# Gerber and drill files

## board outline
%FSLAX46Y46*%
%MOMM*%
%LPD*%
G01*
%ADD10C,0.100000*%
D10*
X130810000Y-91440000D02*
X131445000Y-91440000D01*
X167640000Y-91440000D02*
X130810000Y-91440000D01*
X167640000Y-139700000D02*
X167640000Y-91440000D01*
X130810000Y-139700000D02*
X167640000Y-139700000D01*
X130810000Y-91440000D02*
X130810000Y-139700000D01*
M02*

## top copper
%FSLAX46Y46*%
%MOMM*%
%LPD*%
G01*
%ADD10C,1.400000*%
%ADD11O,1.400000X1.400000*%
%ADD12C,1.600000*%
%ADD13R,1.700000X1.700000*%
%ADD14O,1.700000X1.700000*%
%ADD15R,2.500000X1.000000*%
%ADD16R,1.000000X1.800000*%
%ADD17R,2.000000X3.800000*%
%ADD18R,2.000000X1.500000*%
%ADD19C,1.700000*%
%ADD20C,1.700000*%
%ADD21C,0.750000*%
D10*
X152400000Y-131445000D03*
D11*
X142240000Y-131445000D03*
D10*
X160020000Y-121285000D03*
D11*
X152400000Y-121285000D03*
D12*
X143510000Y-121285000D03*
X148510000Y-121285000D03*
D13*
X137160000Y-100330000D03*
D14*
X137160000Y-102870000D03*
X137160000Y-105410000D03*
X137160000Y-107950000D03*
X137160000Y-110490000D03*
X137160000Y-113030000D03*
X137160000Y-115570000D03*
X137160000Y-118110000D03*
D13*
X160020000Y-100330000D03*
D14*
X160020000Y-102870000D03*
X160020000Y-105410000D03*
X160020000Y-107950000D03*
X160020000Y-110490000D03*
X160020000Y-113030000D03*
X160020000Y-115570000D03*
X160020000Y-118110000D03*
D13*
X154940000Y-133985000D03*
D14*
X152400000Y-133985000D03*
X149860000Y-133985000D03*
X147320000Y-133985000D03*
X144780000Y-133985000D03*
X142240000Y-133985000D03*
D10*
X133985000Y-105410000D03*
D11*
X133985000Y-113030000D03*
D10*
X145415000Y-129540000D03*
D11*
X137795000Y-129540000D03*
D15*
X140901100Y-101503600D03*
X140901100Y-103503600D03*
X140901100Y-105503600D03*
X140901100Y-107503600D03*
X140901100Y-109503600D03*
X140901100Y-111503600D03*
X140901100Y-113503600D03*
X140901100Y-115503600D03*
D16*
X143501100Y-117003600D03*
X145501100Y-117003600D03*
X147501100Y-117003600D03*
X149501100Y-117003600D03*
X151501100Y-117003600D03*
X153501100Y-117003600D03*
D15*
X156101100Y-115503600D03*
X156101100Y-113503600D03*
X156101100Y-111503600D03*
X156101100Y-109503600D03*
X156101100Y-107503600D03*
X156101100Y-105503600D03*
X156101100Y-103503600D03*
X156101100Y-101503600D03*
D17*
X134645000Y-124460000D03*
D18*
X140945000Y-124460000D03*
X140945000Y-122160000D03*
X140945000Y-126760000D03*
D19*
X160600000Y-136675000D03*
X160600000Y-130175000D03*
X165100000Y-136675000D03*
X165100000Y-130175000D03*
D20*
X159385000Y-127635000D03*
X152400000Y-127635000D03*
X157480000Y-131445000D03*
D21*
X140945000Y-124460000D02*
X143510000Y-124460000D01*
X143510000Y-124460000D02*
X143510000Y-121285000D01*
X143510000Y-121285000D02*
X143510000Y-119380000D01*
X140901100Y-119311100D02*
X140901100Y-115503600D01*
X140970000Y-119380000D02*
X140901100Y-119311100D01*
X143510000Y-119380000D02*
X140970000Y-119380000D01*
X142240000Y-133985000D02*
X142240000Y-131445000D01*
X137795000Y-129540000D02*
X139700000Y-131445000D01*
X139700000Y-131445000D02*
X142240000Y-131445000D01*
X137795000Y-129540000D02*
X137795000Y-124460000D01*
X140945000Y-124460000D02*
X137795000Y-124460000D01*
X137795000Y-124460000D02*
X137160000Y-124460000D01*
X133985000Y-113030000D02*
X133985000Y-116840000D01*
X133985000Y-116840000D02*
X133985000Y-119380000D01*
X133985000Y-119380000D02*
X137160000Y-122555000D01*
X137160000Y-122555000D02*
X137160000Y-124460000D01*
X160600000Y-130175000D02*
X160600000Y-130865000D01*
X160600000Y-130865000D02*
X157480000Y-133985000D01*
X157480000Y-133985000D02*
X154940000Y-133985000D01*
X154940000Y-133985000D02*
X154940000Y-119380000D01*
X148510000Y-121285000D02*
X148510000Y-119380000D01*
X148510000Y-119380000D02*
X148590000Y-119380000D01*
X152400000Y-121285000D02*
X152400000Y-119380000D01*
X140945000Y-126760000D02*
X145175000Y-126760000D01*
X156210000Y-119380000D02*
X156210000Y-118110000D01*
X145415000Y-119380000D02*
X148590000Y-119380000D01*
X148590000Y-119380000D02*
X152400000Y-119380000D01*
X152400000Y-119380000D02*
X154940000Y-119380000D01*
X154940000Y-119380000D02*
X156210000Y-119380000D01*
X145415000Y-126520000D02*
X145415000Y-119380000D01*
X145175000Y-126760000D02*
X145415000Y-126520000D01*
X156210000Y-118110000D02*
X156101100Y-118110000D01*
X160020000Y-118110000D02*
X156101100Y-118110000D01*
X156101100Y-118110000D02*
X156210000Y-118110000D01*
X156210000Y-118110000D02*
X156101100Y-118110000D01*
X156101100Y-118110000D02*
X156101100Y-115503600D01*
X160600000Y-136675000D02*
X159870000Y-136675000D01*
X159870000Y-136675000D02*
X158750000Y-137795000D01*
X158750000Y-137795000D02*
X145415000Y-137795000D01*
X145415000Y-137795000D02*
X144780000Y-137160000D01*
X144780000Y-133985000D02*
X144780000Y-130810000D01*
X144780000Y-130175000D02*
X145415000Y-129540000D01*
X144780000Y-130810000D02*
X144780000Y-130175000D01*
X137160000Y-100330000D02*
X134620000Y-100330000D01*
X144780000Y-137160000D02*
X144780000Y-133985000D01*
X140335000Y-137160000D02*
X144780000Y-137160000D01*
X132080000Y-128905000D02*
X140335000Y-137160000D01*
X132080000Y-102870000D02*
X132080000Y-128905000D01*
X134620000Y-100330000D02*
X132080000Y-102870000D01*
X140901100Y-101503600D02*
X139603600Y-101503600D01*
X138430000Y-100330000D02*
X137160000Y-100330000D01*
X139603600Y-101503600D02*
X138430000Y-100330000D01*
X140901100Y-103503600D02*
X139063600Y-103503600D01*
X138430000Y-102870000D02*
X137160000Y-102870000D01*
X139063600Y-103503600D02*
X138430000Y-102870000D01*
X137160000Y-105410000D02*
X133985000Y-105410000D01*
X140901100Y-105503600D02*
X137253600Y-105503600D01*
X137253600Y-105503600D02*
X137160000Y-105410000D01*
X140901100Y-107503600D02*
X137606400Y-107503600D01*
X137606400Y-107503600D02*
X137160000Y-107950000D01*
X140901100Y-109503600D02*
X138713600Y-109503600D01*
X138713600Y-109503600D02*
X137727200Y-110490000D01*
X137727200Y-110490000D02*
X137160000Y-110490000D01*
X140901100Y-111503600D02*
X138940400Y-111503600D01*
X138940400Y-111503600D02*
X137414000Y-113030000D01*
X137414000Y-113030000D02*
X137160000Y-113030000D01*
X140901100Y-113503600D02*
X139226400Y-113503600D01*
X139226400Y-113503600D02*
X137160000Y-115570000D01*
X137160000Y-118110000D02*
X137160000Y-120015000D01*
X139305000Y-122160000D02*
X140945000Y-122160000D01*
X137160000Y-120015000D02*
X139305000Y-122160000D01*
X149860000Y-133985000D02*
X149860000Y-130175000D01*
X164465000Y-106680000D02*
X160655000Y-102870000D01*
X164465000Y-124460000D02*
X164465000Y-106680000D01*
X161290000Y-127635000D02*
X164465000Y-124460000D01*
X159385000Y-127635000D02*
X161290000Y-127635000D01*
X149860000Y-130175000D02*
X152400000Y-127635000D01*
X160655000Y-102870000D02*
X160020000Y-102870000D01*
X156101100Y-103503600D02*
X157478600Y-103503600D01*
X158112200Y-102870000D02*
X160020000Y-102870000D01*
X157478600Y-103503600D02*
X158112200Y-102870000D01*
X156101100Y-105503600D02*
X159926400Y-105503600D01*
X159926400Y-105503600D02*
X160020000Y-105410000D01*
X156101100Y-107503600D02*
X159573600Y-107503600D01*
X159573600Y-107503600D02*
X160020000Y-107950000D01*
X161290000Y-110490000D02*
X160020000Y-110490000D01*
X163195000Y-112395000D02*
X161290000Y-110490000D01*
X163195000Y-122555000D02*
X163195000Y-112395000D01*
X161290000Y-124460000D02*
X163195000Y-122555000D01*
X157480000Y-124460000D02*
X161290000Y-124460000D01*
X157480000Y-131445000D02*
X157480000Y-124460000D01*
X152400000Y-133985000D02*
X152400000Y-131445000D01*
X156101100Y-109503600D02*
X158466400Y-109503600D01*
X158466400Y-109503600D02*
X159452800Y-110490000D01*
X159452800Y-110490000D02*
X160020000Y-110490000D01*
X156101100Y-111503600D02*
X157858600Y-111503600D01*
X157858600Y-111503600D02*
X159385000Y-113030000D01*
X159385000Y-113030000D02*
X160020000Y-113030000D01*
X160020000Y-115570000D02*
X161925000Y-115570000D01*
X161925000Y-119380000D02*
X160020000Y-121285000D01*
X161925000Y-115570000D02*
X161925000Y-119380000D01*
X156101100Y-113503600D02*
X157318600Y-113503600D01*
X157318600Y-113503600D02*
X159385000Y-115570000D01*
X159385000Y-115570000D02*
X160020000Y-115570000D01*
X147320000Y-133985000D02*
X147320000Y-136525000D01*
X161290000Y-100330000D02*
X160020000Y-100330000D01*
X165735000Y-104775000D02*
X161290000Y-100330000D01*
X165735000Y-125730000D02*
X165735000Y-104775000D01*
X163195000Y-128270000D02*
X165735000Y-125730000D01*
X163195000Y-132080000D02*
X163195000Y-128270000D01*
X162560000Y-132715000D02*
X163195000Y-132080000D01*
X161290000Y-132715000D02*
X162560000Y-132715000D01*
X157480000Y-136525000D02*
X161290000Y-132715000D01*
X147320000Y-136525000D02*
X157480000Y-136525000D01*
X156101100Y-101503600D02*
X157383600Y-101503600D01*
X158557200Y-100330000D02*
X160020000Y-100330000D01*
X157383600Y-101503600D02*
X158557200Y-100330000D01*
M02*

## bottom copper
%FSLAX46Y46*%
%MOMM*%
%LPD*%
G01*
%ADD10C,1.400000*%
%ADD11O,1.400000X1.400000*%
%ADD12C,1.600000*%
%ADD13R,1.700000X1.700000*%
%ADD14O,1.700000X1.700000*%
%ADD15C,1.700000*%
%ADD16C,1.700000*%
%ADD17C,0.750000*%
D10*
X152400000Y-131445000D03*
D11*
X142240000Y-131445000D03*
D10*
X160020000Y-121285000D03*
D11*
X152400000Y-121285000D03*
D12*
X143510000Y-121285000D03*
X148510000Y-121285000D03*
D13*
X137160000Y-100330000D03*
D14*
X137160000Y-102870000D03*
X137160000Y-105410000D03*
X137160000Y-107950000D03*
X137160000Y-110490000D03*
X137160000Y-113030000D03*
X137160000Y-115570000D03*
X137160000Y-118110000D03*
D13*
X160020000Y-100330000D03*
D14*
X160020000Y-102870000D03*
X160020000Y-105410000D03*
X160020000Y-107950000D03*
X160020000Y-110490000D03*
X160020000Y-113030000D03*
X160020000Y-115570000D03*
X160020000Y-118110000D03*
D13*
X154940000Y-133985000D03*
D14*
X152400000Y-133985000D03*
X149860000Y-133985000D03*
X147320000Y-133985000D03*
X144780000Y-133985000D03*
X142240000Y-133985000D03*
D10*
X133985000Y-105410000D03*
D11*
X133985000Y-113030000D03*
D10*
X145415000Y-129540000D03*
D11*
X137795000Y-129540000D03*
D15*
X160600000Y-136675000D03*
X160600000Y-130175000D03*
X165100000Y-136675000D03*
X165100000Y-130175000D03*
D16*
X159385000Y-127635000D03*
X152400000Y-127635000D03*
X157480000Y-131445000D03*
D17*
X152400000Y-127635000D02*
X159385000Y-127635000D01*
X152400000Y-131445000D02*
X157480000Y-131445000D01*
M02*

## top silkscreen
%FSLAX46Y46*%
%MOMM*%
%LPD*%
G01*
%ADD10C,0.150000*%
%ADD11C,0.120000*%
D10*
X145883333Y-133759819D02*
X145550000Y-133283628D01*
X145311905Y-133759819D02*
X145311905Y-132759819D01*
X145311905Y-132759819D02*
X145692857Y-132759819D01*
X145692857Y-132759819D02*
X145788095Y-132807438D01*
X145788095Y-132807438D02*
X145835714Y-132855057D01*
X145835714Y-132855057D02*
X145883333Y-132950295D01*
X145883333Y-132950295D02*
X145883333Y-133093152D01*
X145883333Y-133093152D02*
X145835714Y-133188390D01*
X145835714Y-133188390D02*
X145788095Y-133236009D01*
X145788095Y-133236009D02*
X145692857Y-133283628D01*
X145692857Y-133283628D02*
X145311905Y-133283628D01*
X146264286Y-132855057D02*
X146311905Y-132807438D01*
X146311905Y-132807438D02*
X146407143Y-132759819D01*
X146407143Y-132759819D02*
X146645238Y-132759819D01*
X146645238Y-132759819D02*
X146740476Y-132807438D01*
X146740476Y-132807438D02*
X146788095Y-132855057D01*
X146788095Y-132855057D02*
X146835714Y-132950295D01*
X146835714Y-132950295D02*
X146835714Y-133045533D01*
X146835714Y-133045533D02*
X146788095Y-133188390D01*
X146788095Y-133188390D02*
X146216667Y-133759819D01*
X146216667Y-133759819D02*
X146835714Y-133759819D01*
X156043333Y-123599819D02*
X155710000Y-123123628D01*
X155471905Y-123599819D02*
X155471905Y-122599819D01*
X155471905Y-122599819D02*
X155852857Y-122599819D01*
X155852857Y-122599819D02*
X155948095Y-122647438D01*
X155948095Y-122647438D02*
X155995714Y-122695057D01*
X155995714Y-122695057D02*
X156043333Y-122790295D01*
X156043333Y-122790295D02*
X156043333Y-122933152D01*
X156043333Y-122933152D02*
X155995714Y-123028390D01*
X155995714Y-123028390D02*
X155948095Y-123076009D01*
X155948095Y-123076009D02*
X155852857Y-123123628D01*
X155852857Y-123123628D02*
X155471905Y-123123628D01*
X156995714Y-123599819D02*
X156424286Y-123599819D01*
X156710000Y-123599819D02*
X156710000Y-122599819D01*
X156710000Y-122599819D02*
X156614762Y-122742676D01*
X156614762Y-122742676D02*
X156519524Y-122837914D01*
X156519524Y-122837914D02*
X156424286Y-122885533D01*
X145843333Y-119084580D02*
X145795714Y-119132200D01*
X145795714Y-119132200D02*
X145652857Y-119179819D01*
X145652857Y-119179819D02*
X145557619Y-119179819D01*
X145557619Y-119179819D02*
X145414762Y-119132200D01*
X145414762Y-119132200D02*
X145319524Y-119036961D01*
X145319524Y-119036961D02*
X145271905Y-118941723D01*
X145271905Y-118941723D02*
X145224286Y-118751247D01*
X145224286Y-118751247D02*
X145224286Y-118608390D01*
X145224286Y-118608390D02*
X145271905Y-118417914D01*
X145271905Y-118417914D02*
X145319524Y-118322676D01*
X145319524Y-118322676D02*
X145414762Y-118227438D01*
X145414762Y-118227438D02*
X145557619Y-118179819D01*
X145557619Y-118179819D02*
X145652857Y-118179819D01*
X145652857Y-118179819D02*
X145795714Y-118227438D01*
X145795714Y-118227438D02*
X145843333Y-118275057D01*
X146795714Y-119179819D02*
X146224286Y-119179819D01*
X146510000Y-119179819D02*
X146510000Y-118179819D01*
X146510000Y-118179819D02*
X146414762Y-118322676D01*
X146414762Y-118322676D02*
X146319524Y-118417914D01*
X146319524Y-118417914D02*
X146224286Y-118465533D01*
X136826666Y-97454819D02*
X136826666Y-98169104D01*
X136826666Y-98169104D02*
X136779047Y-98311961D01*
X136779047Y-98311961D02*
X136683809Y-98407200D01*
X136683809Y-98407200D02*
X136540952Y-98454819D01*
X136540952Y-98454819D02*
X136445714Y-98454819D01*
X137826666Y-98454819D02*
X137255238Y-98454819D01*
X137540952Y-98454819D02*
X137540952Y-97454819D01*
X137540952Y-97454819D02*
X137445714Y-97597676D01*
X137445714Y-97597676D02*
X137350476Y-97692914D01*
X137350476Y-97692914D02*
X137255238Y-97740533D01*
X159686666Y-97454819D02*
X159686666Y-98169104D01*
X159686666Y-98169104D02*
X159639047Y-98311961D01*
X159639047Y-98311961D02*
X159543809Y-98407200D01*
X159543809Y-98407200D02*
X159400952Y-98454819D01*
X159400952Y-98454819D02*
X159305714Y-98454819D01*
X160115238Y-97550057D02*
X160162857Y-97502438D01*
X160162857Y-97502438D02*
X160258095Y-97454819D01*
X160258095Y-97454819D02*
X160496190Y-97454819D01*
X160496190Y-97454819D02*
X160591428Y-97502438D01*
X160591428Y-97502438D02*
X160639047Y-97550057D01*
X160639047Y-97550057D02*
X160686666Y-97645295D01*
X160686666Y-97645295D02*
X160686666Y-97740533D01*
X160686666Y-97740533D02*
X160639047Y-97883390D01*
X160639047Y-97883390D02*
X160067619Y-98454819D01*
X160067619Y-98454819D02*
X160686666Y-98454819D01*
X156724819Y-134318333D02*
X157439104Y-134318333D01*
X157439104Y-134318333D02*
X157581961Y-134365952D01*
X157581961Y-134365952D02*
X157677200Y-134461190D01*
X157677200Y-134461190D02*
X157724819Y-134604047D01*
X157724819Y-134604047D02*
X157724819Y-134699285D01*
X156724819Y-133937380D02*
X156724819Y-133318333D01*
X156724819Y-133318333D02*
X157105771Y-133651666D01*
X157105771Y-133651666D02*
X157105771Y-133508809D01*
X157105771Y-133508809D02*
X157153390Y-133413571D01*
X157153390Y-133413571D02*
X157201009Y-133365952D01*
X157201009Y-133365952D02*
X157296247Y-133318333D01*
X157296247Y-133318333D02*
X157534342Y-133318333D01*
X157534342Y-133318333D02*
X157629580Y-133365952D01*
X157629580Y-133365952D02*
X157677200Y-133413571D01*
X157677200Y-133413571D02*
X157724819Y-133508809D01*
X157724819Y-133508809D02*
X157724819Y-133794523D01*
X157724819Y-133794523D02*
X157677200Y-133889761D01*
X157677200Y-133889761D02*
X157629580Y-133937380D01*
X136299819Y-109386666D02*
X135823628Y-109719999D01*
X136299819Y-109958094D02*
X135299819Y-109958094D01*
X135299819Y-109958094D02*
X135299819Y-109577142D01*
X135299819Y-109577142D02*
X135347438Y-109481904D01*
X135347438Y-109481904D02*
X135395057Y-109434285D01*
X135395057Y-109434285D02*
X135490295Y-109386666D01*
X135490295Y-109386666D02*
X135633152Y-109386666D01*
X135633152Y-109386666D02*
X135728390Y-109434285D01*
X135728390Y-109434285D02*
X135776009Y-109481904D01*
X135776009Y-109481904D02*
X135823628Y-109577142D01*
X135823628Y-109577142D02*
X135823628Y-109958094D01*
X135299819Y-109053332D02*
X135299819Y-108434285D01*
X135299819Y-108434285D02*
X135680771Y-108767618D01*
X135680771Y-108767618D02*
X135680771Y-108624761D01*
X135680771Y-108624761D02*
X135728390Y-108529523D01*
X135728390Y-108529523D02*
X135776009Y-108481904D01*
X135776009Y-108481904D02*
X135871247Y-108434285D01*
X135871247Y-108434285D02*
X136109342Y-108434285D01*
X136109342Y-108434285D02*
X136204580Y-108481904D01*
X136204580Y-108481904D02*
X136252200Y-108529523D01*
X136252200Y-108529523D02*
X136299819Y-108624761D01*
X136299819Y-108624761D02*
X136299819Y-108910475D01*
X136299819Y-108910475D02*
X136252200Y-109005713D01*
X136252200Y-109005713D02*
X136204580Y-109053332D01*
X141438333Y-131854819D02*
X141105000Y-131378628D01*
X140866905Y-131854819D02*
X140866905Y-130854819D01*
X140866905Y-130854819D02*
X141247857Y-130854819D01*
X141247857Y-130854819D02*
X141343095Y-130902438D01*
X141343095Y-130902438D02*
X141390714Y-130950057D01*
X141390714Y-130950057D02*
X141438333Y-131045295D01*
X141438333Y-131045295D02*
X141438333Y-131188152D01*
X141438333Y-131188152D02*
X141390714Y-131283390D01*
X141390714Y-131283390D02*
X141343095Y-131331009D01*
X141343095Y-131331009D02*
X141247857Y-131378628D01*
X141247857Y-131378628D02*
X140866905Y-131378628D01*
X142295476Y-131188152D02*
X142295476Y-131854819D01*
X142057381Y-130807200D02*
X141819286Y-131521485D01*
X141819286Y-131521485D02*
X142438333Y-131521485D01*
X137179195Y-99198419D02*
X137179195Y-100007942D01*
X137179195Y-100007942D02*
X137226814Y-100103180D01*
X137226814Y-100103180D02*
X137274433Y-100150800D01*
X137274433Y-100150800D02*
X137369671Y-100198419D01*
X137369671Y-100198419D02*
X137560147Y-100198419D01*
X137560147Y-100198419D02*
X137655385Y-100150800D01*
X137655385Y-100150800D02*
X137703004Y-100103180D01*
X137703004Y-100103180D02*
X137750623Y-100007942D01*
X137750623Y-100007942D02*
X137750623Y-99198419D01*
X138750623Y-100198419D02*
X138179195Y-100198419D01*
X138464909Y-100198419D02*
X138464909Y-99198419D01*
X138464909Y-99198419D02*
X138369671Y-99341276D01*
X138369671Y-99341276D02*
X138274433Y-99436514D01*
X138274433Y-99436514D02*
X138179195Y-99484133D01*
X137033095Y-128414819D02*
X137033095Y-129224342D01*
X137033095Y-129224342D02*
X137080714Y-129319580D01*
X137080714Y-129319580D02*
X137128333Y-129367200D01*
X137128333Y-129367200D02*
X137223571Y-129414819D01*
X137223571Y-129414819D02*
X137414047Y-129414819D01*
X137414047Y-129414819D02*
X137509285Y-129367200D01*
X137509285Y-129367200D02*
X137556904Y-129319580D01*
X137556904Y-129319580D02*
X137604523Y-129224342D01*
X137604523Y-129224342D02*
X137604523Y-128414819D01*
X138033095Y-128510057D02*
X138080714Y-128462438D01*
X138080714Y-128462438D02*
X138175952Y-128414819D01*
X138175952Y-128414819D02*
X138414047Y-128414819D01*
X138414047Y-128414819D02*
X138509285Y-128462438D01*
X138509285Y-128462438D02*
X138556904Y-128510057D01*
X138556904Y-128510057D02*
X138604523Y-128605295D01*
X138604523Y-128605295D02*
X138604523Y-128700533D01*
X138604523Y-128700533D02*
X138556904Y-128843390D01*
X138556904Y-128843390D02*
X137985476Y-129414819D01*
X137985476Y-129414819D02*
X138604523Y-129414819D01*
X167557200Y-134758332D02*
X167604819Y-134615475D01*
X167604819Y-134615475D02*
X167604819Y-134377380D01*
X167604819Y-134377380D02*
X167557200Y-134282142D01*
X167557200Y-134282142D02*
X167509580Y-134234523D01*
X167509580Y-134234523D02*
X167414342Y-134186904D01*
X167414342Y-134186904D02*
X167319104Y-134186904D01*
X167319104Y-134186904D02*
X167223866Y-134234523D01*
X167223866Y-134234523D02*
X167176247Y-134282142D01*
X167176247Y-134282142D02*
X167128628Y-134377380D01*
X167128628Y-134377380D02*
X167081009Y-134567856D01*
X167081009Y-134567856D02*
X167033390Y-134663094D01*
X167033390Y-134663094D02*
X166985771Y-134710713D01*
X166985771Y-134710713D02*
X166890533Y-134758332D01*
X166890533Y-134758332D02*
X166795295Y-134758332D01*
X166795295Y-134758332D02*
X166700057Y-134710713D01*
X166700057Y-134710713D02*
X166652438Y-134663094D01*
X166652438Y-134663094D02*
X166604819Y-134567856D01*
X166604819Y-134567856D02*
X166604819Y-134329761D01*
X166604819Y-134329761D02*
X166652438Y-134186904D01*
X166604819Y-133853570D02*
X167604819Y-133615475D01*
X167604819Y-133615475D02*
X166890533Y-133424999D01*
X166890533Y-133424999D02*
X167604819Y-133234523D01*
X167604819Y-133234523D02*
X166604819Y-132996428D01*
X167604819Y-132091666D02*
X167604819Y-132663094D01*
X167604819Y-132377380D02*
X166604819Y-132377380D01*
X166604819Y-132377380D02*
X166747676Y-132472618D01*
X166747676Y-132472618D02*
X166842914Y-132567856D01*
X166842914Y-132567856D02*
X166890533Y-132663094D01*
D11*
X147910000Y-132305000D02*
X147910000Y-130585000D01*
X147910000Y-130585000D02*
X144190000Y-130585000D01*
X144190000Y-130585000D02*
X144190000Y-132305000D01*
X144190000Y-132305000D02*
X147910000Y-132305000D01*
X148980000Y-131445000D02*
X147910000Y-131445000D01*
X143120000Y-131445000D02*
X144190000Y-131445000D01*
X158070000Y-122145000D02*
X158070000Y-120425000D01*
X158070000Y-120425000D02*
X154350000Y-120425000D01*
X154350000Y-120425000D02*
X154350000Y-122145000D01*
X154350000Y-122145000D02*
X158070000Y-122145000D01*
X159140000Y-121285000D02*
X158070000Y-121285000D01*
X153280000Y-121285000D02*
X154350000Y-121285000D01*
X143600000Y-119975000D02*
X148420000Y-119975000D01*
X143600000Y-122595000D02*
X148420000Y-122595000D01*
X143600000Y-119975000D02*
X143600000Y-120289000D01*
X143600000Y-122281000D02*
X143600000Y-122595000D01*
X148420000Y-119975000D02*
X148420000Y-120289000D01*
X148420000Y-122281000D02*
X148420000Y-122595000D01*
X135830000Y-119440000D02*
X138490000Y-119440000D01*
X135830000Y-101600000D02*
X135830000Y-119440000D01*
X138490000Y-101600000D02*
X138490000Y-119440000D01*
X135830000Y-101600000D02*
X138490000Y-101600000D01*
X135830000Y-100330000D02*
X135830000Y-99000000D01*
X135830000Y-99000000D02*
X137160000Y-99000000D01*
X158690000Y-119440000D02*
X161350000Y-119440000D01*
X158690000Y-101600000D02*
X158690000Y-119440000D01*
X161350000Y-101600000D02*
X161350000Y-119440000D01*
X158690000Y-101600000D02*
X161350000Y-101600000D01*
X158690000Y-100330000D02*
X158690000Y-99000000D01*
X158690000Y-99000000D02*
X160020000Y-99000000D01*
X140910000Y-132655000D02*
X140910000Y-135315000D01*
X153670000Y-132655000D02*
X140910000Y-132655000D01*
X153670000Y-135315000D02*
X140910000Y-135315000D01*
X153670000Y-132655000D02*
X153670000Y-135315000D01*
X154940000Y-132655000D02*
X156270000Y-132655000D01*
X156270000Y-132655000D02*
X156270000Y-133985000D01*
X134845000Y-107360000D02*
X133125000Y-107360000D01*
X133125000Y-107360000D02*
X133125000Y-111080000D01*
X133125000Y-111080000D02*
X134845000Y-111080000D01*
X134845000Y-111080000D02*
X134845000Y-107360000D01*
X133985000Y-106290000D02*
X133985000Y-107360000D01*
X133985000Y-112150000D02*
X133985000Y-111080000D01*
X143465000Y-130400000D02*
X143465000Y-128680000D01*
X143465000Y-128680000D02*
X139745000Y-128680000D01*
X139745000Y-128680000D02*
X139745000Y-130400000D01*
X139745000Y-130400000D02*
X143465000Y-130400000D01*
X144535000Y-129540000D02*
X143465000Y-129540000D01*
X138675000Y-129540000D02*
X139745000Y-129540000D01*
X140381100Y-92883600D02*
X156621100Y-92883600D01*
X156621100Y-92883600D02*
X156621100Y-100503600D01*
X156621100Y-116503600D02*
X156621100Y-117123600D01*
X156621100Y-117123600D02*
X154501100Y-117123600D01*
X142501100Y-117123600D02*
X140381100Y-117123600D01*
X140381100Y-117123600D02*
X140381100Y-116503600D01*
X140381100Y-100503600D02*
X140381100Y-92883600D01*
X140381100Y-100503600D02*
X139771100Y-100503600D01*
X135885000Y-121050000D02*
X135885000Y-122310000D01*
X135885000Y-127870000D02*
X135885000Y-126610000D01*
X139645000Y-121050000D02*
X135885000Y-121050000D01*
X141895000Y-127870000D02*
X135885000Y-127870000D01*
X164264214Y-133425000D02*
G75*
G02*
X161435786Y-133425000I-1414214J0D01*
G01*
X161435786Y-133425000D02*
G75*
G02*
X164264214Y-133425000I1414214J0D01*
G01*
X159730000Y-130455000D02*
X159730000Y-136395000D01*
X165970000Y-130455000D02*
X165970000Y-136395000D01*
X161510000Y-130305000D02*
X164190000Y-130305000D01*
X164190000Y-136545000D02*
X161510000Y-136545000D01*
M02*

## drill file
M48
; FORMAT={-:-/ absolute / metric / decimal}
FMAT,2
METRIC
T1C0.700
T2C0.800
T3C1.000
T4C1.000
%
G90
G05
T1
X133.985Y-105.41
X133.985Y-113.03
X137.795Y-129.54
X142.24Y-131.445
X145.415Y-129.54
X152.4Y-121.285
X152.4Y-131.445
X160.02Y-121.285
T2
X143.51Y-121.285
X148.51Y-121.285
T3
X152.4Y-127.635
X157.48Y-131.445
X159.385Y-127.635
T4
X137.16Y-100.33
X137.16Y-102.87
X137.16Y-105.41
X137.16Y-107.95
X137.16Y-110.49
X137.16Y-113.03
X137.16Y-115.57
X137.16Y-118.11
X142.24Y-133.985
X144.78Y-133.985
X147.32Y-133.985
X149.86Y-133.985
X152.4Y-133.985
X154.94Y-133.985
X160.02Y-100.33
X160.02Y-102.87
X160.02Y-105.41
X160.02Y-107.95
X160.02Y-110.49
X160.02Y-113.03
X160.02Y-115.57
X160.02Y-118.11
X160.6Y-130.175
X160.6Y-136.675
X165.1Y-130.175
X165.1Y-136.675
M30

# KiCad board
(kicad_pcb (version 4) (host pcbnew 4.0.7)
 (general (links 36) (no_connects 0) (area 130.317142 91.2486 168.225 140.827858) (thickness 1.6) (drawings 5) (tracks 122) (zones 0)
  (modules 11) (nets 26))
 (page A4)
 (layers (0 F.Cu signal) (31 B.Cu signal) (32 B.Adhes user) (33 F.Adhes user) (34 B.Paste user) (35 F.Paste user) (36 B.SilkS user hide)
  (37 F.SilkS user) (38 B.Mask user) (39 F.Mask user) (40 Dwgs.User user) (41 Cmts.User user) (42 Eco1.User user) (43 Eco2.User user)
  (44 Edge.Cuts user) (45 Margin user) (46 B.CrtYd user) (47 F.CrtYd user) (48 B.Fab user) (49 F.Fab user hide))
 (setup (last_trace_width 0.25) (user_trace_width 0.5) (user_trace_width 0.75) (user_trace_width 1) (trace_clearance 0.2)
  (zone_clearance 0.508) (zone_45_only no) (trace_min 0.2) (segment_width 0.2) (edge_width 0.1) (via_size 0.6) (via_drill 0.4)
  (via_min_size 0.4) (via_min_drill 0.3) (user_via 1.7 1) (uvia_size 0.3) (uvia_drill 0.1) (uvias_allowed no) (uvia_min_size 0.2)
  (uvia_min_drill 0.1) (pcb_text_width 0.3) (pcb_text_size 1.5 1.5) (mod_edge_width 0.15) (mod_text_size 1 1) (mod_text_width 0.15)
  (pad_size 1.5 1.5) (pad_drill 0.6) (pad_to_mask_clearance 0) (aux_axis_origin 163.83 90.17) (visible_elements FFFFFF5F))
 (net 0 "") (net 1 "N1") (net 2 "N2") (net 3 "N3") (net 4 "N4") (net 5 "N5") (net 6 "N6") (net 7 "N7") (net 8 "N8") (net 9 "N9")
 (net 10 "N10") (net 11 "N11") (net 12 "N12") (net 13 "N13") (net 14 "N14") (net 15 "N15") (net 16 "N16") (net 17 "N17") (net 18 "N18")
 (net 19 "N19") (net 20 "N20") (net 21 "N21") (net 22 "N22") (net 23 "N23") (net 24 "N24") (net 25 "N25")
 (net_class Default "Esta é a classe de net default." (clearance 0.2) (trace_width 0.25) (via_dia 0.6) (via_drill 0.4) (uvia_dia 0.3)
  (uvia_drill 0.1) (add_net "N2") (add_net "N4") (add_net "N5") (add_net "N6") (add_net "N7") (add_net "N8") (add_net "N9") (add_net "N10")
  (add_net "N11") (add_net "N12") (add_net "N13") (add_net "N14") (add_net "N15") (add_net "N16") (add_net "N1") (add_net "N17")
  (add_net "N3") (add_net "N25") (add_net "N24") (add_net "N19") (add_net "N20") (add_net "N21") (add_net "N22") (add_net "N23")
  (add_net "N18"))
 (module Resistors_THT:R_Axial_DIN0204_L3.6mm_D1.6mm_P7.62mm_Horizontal (layer F.Cu) (at 149.86 131.445 180)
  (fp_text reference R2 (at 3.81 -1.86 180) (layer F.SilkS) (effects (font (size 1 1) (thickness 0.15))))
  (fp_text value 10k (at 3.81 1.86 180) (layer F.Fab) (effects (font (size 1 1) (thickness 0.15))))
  (fp_line (start 1.95 -0.86) (end 1.95 0.86) (layer F.SilkS) (width 0.12))
  (fp_line (start 1.95 0.86) (end 5.67 0.86) (layer F.SilkS) (width 0.12))
  (fp_line (start 5.67 0.86) (end 5.67 -0.86) (layer F.SilkS) (width 0.12))
  (fp_line (start 5.67 -0.86) (end 1.95 -0.86) (layer F.SilkS) (width 0.12))
  (fp_line (start 0.88 0) (end 1.95 0) (layer F.SilkS) (width 0.12))
  (fp_line (start 6.74 0) (end 5.67 0) (layer F.SilkS) (width 0.12))
  (pad 1 thru_hole circle (at -2.54 0 180) (size 1.4 1.4) (drill 0.7) (layers *.Cu *.Mask) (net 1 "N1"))
  (pad 2 thru_hole oval (at 7.62 0 180) (size 1.4 1.4) (drill 0.7) (layers *.Cu *.Mask) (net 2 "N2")))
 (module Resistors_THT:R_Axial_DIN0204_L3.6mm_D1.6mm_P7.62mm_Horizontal (layer F.Cu) (at 160.02 121.285 180)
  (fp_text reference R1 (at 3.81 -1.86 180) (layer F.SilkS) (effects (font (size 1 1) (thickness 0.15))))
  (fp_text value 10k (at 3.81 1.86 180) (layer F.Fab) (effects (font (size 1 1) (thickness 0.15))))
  (fp_line (start 1.95 -0.86) (end 1.95 0.86) (layer F.SilkS) (width 0.12))
  (fp_line (start 1.95 0.86) (end 5.67 0.86) (layer F.SilkS) (width 0.12))
  (fp_line (start 5.67 0.86) (end 5.67 -0.86) (layer F.SilkS) (width 0.12))
  (fp_line (start 5.67 -0.86) (end 1.95 -0.86) (layer F.SilkS) (width 0.12))
  (fp_line (start 0.88 0) (end 1.95 0) (layer F.SilkS) (width 0.12))
  (fp_line (start 6.74 0) (end 5.67 0) (layer F.SilkS) (width 0.12))
  (pad 1 thru_hole circle (at 0 0 180) (size 1.4 1.4) (drill 0.7) (layers *.Cu *.Mask) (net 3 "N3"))
  (pad 2 thru_hole oval (at 7.62 0 180) (size 1.4 1.4) (drill 0.7) (layers *.Cu *.Mask) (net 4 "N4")))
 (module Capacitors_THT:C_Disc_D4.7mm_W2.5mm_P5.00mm (layer F.Cu) (at 143.51 121.285)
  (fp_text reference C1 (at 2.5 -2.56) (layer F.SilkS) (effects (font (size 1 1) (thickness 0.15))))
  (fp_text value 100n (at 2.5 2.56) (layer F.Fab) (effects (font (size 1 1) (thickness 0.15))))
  (fp_line (start 0.09 -1.31) (end 4.91 -1.31) (layer F.SilkS) (width 0.12))
  (fp_line (start 0.09 1.31) (end 4.91 1.31) (layer F.SilkS) (width 0.12))
  (fp_line (start 0.09 -1.31) (end 0.09 -0.996) (layer F.SilkS) (width 0.12))
  (fp_line (start 0.09 0.996) (end 0.09 1.31) (layer F.SilkS) (width 0.12))
  (fp_line (start 4.91 -1.31) (end 4.91 -0.996) (layer F.SilkS) (width 0.12))
  (fp_line (start 4.91 0.996) (end 4.91 1.31) (layer F.SilkS) (width 0.12))
  (pad 1 thru_hole circle (at 0 0) (size 1.6 1.6) (drill 0.8) (layers *.Cu *.Mask) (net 2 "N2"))
  (pad 2 thru_hole circle (at 5 0) (size 1.6 1.6) (drill 0.8) (layers *.Cu *.Mask) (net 4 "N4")))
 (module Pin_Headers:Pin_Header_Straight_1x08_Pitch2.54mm (layer F.Cu) (at 137.16 100.33)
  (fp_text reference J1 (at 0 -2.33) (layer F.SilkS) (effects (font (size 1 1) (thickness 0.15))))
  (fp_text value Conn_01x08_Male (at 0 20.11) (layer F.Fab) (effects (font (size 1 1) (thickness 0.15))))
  (fp_line (start -1.33 19.11) (end 1.33 19.11) (layer F.SilkS) (width 0.12))
  (fp_line (start -1.33 1.27) (end -1.33 19.11) (layer F.SilkS) (width 0.12))
  (fp_line (start 1.33 1.27) (end 1.33 19.11) (layer F.SilkS) (width 0.12))
  (fp_line (start -1.33 1.27) (end 1.33 1.27) (layer F.SilkS) (width 0.12))
  (fp_line (start -1.33 0) (end -1.33 -1.33) (layer F.SilkS) (width 0.12))
  (fp_line (start -1.33 -1.33) (end 0 -1.33) (layer F.SilkS) (width 0.12))
  (pad 1 thru_hole rect (at 0 0) (size 1.7 1.7) (drill 1) (layers *.Cu *.Mask) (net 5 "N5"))
  (pad 2 thru_hole oval (at 0 2.54) (size 1.7 1.7) (drill 1) (layers *.Cu *.Mask) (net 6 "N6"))
  (pad 3 thru_hole oval (at 0 5.08) (size 1.7 1.7) (drill 1) (layers *.Cu *.Mask) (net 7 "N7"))
  (pad 4 thru_hole oval (at 0 7.62) (size 1.7 1.7) (drill 1) (layers *.Cu *.Mask) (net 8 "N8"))
  (pad 5 thru_hole oval (at 0 10.16) (size 1.7 1.7) (drill 1) (layers *.Cu *.Mask) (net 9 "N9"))
  (pad 6 thru_hole oval (at 0 12.7) (size 1.7 1.7) (drill 1) (layers *.Cu *.Mask) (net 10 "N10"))
  (pad 7 thru_hole oval (at 0 15.24) (size 1.7 1.7) (drill 1) (layers *.Cu *.Mask) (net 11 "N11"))
  (pad 8 thru_hole oval (at 0 17.78) (size 1.7 1.7) (drill 1) (layers *.Cu *.Mask) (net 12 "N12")))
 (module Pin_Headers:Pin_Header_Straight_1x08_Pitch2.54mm (layer F.Cu) (at 160.02 100.33)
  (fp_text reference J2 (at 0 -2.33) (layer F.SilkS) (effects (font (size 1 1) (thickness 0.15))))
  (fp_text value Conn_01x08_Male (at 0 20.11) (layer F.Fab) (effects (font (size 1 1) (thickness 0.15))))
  (fp_line (start -1.33 19.11) (end 1.33 19.11) (layer F.SilkS) (width 0.12))
  (fp_line (start -1.33 1.27) (end -1.33 19.11) (layer F.SilkS) (width 0.12))
  (fp_line (start 1.33 1.27) (end 1.33 19.11) (layer F.SilkS) (width 0.12))
  (fp_line (start -1.33 1.27) (end 1.33 1.27) (layer F.SilkS) (width 0.12))
  (fp_line (start -1.33 0) (end -1.33 -1.33) (layer F.SilkS) (width 0.12))
  (fp_line (start -1.33 -1.33) (end 0 -1.33) (layer F.SilkS) (width 0.12))
  (pad 1 thru_hole rect (at 0 0) (size 1.7 1.7) (drill 1) (layers *.Cu *.Mask) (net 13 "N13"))
  (pad 2 thru_hole oval (at 0 2.54) (size 1.7 1.7) (drill 1) (layers *.Cu *.Mask) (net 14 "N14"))
  (pad 3 thru_hole oval (at 0 5.08) (size 1.7 1.7) (drill 1) (layers *.Cu *.Mask) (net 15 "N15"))
  (pad 4 thru_hole oval (at 0 7.62) (size 1.7 1.7) (drill 1) (layers *.Cu *.Mask) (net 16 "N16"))
  (pad 5 thru_hole oval (at 0 10.16) (size 1.7 1.7) (drill 1) (layers *.Cu *.Mask) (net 1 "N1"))
  (pad 6 thru_hole oval (at 0 12.7) (size 1.7 1.7) (drill 1) (layers *.Cu *.Mask) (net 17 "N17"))
  (pad 7 thru_hole oval (at 0 15.24) (size 1.7 1.7) (drill 1) (layers *.Cu *.Mask) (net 3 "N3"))
  (pad 8 thru_hole oval (at 0 17.78) (size 1.7 1.7) (drill 1) (layers *.Cu *.Mask) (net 4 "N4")))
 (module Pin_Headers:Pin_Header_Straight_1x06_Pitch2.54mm (layer F.Cu) (at 154.94 133.985 270)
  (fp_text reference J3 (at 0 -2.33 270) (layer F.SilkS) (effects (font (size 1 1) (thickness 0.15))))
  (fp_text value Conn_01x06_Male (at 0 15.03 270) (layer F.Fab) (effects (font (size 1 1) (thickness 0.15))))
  (fp_line (start -1.33 14.03) (end 1.33 14.03) (layer F.SilkS) (width 0.12))
  (fp_line (start -1.33 1.27) (end -1.33 14.03) (layer F.SilkS) (width 0.12))
  (fp_line (start 1.33 1.27) (end 1.33 14.03) (layer F.SilkS) (width 0.12))
  (fp_line (start -1.33 1.27) (end 1.33 1.27) (layer F.SilkS) (width 0.12))
  (fp_line (start -1.33 0) (end -1.33 -1.33) (layer F.SilkS) (width 0.12))
  (fp_line (start -1.33 -1.33) (end 0 -1.33) (layer F.SilkS) (width 0.12))
  (pad 1 thru_hole rect (at 0 0 270) (size 1.7 1.7) (drill 1) (layers *.Cu *.Mask) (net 4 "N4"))
  (pad 2 thru_hole oval (at 0 2.54 270) (size 1.7 1.7) (drill 1) (layers *.Cu *.Mask) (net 1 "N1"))
  (pad 3 thru_hole oval (at 0 5.08 270) (size 1.7 1.7) (drill 1) (layers *.Cu *.Mask) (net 14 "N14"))
  (pad 4 thru_hole oval (at 0 7.62 270) (size 1.7 1.7) (drill 1) (layers *.Cu *.Mask) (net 13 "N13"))
  (pad 5 thru_hole oval (at 0 10.16 270) (size 1.7 1.7) (drill 1) (layers *.Cu *.Mask) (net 5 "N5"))
  (pad 6 thru_hole oval (at 0 12.7 270) (size 1.7 1.7) (drill 1) (layers *.Cu *.Mask) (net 2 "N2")))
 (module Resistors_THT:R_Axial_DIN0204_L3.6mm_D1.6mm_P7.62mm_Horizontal (layer F.Cu) (at 133.985 105.41 270)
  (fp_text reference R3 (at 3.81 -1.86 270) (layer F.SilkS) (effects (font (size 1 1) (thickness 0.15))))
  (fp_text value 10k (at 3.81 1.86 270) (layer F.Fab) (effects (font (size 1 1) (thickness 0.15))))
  (fp_line (start 1.95 -0.86) (end 1.95 0.86) (layer F.SilkS) (width 0.12))
  (fp_line (start 1.95 0.86) (end 5.67 0.86) (layer F.SilkS) (width 0.12))
  (fp_line (start 5.67 0.86) (end 5.67 -0.86) (layer F.SilkS) (width 0.12))
  (fp_line (start 5.67 -0.86) (end 1.95 -0.86) (layer F.SilkS) (width 0.12))
  (fp_line (start 0.88 0) (end 1.95 0) (layer F.SilkS) (width 0.12))
  (fp_line (start 6.74 0) (end 5.67 0) (layer F.SilkS) (width 0.12))
  (pad 1 thru_hole circle (at 0 0 270) (size 1.4 1.4) (drill 0.7) (layers *.Cu *.Mask) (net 7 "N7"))
  (pad 2 thru_hole oval (at 7.62 0 270) (size 1.4 1.4) (drill 0.7) (layers *.Cu *.Mask) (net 2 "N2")))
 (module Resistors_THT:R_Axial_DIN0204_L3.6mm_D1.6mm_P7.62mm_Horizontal (layer F.Cu) (at 145.415 129.54 180)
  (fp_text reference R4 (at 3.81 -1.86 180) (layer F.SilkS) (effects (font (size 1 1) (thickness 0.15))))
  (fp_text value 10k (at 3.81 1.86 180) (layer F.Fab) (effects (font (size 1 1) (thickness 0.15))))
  (fp_line (start 1.95 -0.86) (end 1.95 0.86) (layer F.SilkS) (width 0.12))
  (fp_line (start 1.95 0.86) (end 5.67 0.86) (layer F.SilkS) (width 0.12))
  (fp_line (start 5.67 0.86) (end 5.67 -0.86) (layer F.SilkS) (width 0.12))
  (fp_line (start 5.67 -0.86) (end 1.95 -0.86) (layer F.SilkS) (width 0.12))
  (fp_line (start 0.88 0) (end 1.95 0) (layer F.SilkS) (width 0.12))
  (fp_line (start 6.74 0) (end 5.67 0) (layer F.SilkS) (width 0.12))
  (pad 1 thru_hole circle (at 0 0 180) (size 1.4 1.4) (drill 0.7) (layers *.Cu *.Mask) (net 5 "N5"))
  (pad 2 thru_hole oval (at 7.62 0 180) (size 1.4 1.4) (drill 0.7) (layers *.Cu *.Mask) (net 2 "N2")))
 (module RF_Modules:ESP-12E (layer F.Cu) (at 148.5011 105.0036)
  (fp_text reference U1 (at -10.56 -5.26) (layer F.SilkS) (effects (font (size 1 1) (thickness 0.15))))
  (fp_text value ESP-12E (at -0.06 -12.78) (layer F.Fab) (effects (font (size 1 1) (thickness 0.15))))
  (fp_line (start -8.12 -12.12) (end 8.12 -12.12) (layer F.SilkS) (width 0.12))
  (fp_line (start 8.12 -12.12) (end 8.12 -4.5) (layer F.SilkS) (width 0.12))
  (fp_line (start 8.12 11.5) (end 8.12 12.12) (layer F.SilkS) (width 0.12))
  (fp_line (start 8.12 12.12) (end 6 12.12) (layer F.SilkS) (width 0.12))
  (fp_line (start -6 12.12) (end -8.12 12.12) (layer F.SilkS) (width 0.12))
  (fp_line (start -8.12 12.12) (end -8.12 11.5) (layer F.SilkS) (width 0.12))
  (fp_line (start -8.12 -4.5) (end -8.12 -12.12) (layer F.SilkS) (width 0.12))
  (fp_line (start -8.12 -4.5) (end -8.73 -4.5) (layer F.SilkS) (width 0.12))
  (pad 1 smd rect (at -7.6 -3.5) (size 2.5 1) (layers F.Cu F.Paste F.Mask) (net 5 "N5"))
  (pad 2 smd rect (at -7.6 -1.5) (size 2.5 1) (layers F.Cu F.Paste F.Mask) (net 6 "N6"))
  (pad 3 smd rect (at -7.6 0.5) (size 2.5 1) (layers F.Cu F.Paste F.Mask) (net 7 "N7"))
  (pad 4 smd rect (at -7.6 2.5) (size 2.5 1) (layers F.Cu F.Paste F.Mask) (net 8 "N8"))
  (pad 5 smd rect (at -7.6 4.5) (size 2.5 1) (layers F.Cu F.Paste F.Mask) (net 9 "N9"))
  (pad 6 smd rect (at -7.6 6.5) (size 2.5 1) (layers F.Cu F.Paste F.Mask) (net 10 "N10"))
  (pad 7 smd rect (at -7.6 8.5) (size 2.5 1) (layers F.Cu F.Paste F.Mask) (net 11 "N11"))
  (pad 8 smd rect (at -7.6 10.5) (size 2.5 1) (layers F.Cu F.Paste F.Mask) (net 2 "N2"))
  (pad 9 smd rect (at -5 12) (size 1 1.8) (layers F.Cu F.Paste F.Mask) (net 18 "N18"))
  (pad 10 smd rect (at -3 12) (size 1 1.8) (layers F.Cu F.Paste F.Mask) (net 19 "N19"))
  (pad 11 smd rect (at -1 12) (size 1 1.8) (layers F.Cu F.Paste F.Mask) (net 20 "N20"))
  (pad 12 smd rect (at 1 12) (size 1 1.8) (layers F.Cu F.Paste F.Mask) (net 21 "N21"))
  (pad 13 smd rect (at 3 12) (size 1 1.8) (layers F.Cu F.Paste F.Mask) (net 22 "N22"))
  (pad 14 smd rect (at 5 12) (size 1 1.8) (layers F.Cu F.Paste F.Mask) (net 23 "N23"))
  (pad 15 smd rect (at 7.6 10.5) (size 2.5 1) (layers F.Cu F.Paste F.Mask) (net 4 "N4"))
  (pad 16 smd rect (at 7.6 8.5) (size 2.5 1) (layers F.Cu F.Paste F.Mask) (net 3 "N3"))
  (pad 17 smd rect (at 7.6 6.5) (size 2.5 1) (layers F.Cu F.Paste F.Mask) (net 17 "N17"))
  (pad 18 smd rect (at 7.6 4.5) (size 2.5 1) (layers F.Cu F.Paste F.Mask) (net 1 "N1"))
  (pad 19 smd rect (at 7.6 2.5) (size 2.5 1) (layers F.Cu F.Paste F.Mask) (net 16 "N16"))
  (pad 20 smd rect (at 7.6 0.5) (size 2.5 1) (layers F.Cu F.Paste F.Mask) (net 15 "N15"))
  (pad 21 smd rect (at 7.6 -1.5) (size 2.5 1) (layers F.Cu F.Paste F.Mask) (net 14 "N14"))
  (pad 22 smd rect (at 7.6 -3.5) (size 2.5 1) (layers F.Cu F.Paste F.Mask) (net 13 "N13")))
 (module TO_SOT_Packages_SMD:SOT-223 (layer F.Cu) (at 137.795 124.46 180)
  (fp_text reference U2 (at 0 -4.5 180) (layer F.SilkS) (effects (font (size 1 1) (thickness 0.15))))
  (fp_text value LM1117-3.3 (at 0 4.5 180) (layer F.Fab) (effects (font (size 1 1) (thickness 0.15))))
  (fp_line (start 1.91 3.41) (end 1.91 2.15) (layer F.SilkS) (width 0.12))
  (fp_line (start 1.91 -3.41) (end 1.91 -2.15) (layer F.SilkS) (width 0.12))
  (fp_line (start -1.85 3.41) (end 1.91 3.41) (layer F.SilkS) (width 0.12))
  (fp_line (start -4.1 -3.41) (end 1.91 -3.41) (layer F.SilkS) (width 0.12))
  (pad 4 smd rect (at 3.15 0 180) (size 2 3.8) (layers F.Cu F.Paste F.Mask))
  (pad 2 smd rect (at -3.15 0 180) (size 2 1.5) (layers F.Cu F.Paste F.Mask) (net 2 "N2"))
  (pad 3 smd rect (at -3.15 2.3 180) (size 2 1.5) (layers F.Cu F.Paste F.Mask) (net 12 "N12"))
  (pad 1 smd rect (at -3.15 -2.3 180) (size 2 1.5) (layers F.Cu F.Paste F.Mask) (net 4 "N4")))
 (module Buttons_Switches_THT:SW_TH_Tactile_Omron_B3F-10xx (layer F.Cu) (at 165.1 130.175 270)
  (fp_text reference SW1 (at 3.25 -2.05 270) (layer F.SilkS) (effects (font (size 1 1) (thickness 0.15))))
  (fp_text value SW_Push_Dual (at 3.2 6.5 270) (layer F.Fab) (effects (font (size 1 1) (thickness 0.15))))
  (fp_circle (center 3.25 2.25) (end 4.25 3.25) (layer F.SilkS) (width 0.12))
  (fp_line (start 0.28 5.37) (end 6.22 5.37) (layer F.SilkS) (width 0.12))
  (fp_line (start 0.28 -0.87) (end 6.22 -0.87) (layer F.SilkS) (width 0.12))
  (fp_line (start 0.13 3.59) (end 0.13 0.91) (layer F.SilkS) (width 0.12))
  (fp_line (start 6.37 0.91) (end 6.37 3.59) (layer F.SilkS) (width 0.12))
  (pad 4 thru_hole circle (at 6.5 4.5 270) (size 1.7 1.7) (drill 1) (layers *.Cu *.Mask) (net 5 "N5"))
  (pad 3 thru_hole circle (at 0 4.5 270) (size 1.7 1.7) (drill 1) (layers *.Cu *.Mask) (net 4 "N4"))
  (pad 2 thru_hole circle (at 6.5 0 270) (size 1.7 1.7) (drill 1) (layers *.Cu *.Mask) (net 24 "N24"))
  (pad 1 thru_hole circle (at 0 0 270) (size 1.7 1.7) (drill 1) (layers *.Cu *.Mask) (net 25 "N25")))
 (gr_line (start 130.81 91.44) (end 131.445 91.44) (angle 90) (layer Edge.Cuts) (width 0.1))
 (gr_line (start 167.64 91.44) (end 130.81 91.44) (angle 90) (layer Edge.Cuts) (width 0.1))
 (gr_line (start 167.64 139.7) (end 167.64 91.44) (angle 90) (layer Edge.Cuts) (width 0.1))
 (gr_line (start 130.81 139.7) (end 167.64 139.7) (angle 90) (layer Edge.Cuts) (width 0.1))
 (gr_line (start 130.81 91.44) (end 130.81 139.7) (angle 90) (layer Edge.Cuts) (width 0.1))
 (segment (start 140.945 124.46) (end 143.51 124.46) (width 0.75) (layer F.Cu) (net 2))
 (segment (start 143.51 124.46) (end 143.51 121.285) (width 0.75) (layer F.Cu) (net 2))
 (segment (start 143.51 121.285) (end 143.51 119.38) (width 0.75) (layer F.Cu) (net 2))
 (segment (start 140.9011 119.3111) (end 140.9011 115.5036) (width 0.75) (layer F.Cu) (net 2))
 (segment (start 140.97 119.38) (end 140.9011 119.3111) (width 0.75) (layer F.Cu) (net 2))
 (segment (start 143.51 119.38) (end 140.97 119.38) (width 0.75) (layer F.Cu) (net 2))
 (segment (start 142.24 133.985) (end 142.24 131.445) (width 0.75) (layer F.Cu) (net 2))
 (segment (start 137.795 129.54) (end 139.7 131.445) (width 0.75) (layer F.Cu) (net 2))
 (segment (start 139.7 131.445) (end 142.24 131.445) (width 0.75) (layer F.Cu) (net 2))
 (segment (start 137.795 129.54) (end 137.795 124.46) (width 0.75) (layer F.Cu) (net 2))
 (segment (start 140.945 124.46) (end 137.795 124.46) (width 0.75) (layer F.Cu) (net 2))
 (segment (start 137.795 124.46) (end 137.16 124.46) (width 0.75) (layer F.Cu) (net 2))
 (segment (start 133.985 113.03) (end 133.985 116.84) (width 0.75) (layer F.Cu) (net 2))
 (segment (start 133.985 116.84) (end 133.985 119.38) (width 0.75) (layer F.Cu) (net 2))
 (segment (start 133.985 119.38) (end 137.16 122.555) (width 0.75) (layer F.Cu) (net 2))
 (segment (start 137.16 122.555) (end 137.16 124.46) (width 0.75) (layer F.Cu) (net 2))
 (segment (start 160.6 130.175) (end 160.6 130.865) (width 0.75) (layer F.Cu) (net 4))
 (segment (start 160.6 130.865) (end 157.48 133.985) (width 0.75) (layer F.Cu) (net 4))
 (segment (start 157.48 133.985) (end 154.94 133.985) (width 0.75) (layer F.Cu) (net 4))
 (segment (start 154.94 133.985) (end 154.94 119.38) (width 0.75) (layer F.Cu) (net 4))
 (segment (start 148.51 121.285) (end 148.51 119.38) (width 0.75) (layer F.Cu) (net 4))
 (segment (start 148.51 119.38) (end 148.59 119.38) (width 0.75) (layer F.Cu) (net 4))
 (segment (start 152.4 121.285) (end 152.4 119.38) (width 0.75) (layer F.Cu) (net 4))
 (segment (start 140.945 126.76) (end 145.175 126.76) (width 0.75) (layer F.Cu) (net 4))
 (segment (start 156.21 119.38) (end 156.21 118.11) (width 0.75) (layer F.Cu) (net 4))
 (segment (start 145.415 119.38) (end 148.59 119.38) (width 0.75) (layer F.Cu) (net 4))
 (segment (start 148.59 119.38) (end 152.4 119.38) (width 0.75) (layer F.Cu) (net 4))
 (segment (start 152.4 119.38) (end 154.94 119.38) (width 0.75) (layer F.Cu) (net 4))
 (segment (start 154.94 119.38) (end 156.21 119.38) (width 0.75) (layer F.Cu) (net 4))
 (segment (start 145.415 126.52) (end 145.415 119.38) (width 0.75) (layer F.Cu) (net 4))
 (segment (start 145.175 126.76) (end 145.415 126.52) (width 0.75) (layer F.Cu) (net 4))
 (segment (start 156.21 118.11) (end 156.1011 118.11) (width 0.75) (layer F.Cu) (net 4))
 (segment (start 160.02 118.11) (end 156.1011 118.11) (width 0.75) (layer F.Cu) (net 4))
 (segment (start 156.1011 118.11) (end 156.21 118.11) (width 0.75) (layer F.Cu) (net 4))
 (segment (start 156.21 118.11) (end 156.1011 118.11) (width 0.75) (layer F.Cu) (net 4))
 (segment (start 156.1011 118.11) (end 156.1011 115.5036) (width 0.75) (layer F.Cu) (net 4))
 (segment (start 160.6 136.675) (end 159.87 136.675) (width 0.75) (layer F.Cu) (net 5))
 (segment (start 159.87 136.675) (end 158.75 137.795) (width 0.75) (layer F.Cu) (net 5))
 (segment (start 158.75 137.795) (end 145.415 137.795) (width 0.75) (layer F.Cu) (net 5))
 (segment (start 145.415 137.795) (end 144.78 137.16) (width 0.75) (layer F.Cu) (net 5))
 (segment (start 144.78 133.985) (end 144.78 130.81) (width 0.75) (layer F.Cu) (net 5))
 (segment (start 144.78 130.175) (end 145.415 129.54) (width 0.75) (layer F.Cu) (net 5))
 (segment (start 144.78 130.81) (end 144.78 130.175) (width 0.75) (layer F.Cu) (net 5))
 (segment (start 137.16 100.33) (end 134.62 100.33) (width 0.75) (layer F.Cu) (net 5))
 (segment (start 144.78 137.16) (end 144.78 133.985) (width 0.75) (layer F.Cu) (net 5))
 (segment (start 140.335 137.16) (end 144.78 137.16) (width 0.75) (layer F.Cu) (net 5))
 (segment (start 132.08 128.905) (end 140.335 137.16) (width 0.75) (layer F.Cu) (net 5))
 (segment (start 132.08 102.87) (end 132.08 128.905) (width 0.75) (layer F.Cu) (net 5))
 (segment (start 134.62 100.33) (end 132.08 102.87) (width 0.75) (layer F.Cu) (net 5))
 (segment (start 140.9011 101.5036) (end 139.6036 101.5036) (width 0.75) (layer F.Cu) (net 5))
 (segment (start 138.43 100.33) (end 137.16 100.33) (width 0.75) (layer F.Cu) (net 5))
 (segment (start 139.6036 101.5036) (end 138.43 100.33) (width 0.75) (layer F.Cu) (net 5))
 (segment (start 140.9011 103.5036) (end 139.0636 103.5036) (width 0.75) (layer F.Cu) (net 6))
 (segment (start 138.43 102.87) (end 137.16 102.87) (width 0.75) (layer F.Cu) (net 6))
 (segment (start 139.0636 103.5036) (end 138.43 102.87) (width 0.75) (layer F.Cu) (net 6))
 (segment (start 137.16 105.41) (end 133.985 105.41) (width 0.75) (layer F.Cu) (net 7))
 (segment (start 140.9011 105.5036) (end 137.2536 105.5036) (width 0.75) (layer F.Cu) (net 7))
 (segment (start 137.2536 105.5036) (end 137.16 105.41) (width 0.75) (layer F.Cu) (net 7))
 (segment (start 140.9011 107.5036) (end 137.6064 107.5036) (width 0.75) (layer F.Cu) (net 8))
 (segment (start 137.6064 107.5036) (end 137.16 107.95) (width 0.75) (layer F.Cu) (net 8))
 (segment (start 140.9011 109.5036) (end 138.7136 109.5036) (width 0.75) (layer F.Cu) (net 9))
 (segment (start 138.7136 109.5036) (end 137.7272 110.49) (width 0.75) (layer F.Cu) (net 9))
 (segment (start 137.7272 110.49) (end 137.16 110.49) (width 0.75) (layer F.Cu) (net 9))
 (segment (start 140.9011 111.5036) (end 138.9404 111.5036) (width 0.75) (layer F.Cu) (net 10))
 (segment (start 138.9404 111.5036) (end 137.414 113.03) (width 0.75) (layer F.Cu) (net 10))
 (segment (start 137.414 113.03) (end 137.16 113.03) (width 0.75) (layer F.Cu) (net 10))
 (segment (start 140.9011 113.5036) (end 139.2264 113.5036) (width 0.75) (layer F.Cu) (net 11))
 (segment (start 139.2264 113.5036) (end 137.16 115.57) (width 0.75) (layer F.Cu) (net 11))
 (segment (start 137.16 118.11) (end 137.16 120.015) (width 0.75) (layer F.Cu) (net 12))
 (segment (start 139.305 122.16) (end 140.945 122.16) (width 0.75) (layer F.Cu) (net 12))
 (segment (start 137.16 120.015) (end 139.305 122.16) (width 0.75) (layer F.Cu) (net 12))
 (segment (start 149.86 133.985) (end 149.86 130.175) (width 0.75) (layer F.Cu) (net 14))
 (segment (start 164.465 106.68) (end 160.655 102.87) (width 0.75) (layer F.Cu) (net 14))
 (segment (start 164.465 124.46) (end 164.465 106.68) (width 0.75) (layer F.Cu) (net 14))
 (segment (start 161.29 127.635) (end 164.465 124.46) (width 0.75) (layer F.Cu) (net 14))
 (segment (start 159.385 127.635) (end 161.29 127.635) (width 0.75) (layer F.Cu) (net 14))
 (via (at 159.385 127.635) (size 1.7) (drill 1) (layers F.Cu B.Cu) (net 14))
 (segment (start 152.4 127.635) (end 159.385 127.635) (width 0.75) (layer B.Cu) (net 14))
 (via (at 152.4 127.635) (size 1.7) (drill 1) (layers F.Cu B.Cu) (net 14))
 (segment (start 149.86 130.175) (end 152.4 127.635) (width 0.75) (layer F.Cu) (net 14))
 (segment (start 160.655 102.87) (end 160.02 102.87) (width 0.75) (layer F.Cu) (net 14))
 (segment (start 156.1011 103.5036) (end 157.4786 103.5036) (width 0.75) (layer F.Cu) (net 14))
 (segment (start 158.1122 102.87) (end 160.02 102.87) (width 0.75) (layer F.Cu) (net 14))
 (segment (start 157.4786 103.5036) (end 158.1122 102.87) (width 0.75) (layer F.Cu) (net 14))
 (segment (start 156.1011 105.5036) (end 159.9264 105.5036) (width 0.75) (layer F.Cu) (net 15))
 (segment (start 159.9264 105.5036) (end 160.02 105.41) (width 0.75) (layer F.Cu) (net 15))
 (segment (start 156.1011 107.5036) (end 159.5736 107.5036) (width 0.75) (layer F.Cu) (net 16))
 (segment (start 159.5736 107.5036) (end 160.02 107.95) (width 0.75) (layer F.Cu) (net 16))
 (segment (start 152.4 131.445) (end 157.48 131.445) (width 0.75) (layer B.Cu) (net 1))
 (segment (start 161.29 110.49) (end 160.02 110.49) (width 0.75) (layer F.Cu) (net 1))
 (segment (start 163.195 112.395) (end 161.29 110.49) (width 0.75) (layer F.Cu) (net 1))
 (segment (start 163.195 122.555) (end 163.195 112.395) (width 0.75) (layer F.Cu) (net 1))
 (segment (start 161.29 124.46) (end 163.195 122.555) (width 0.75) (layer F.Cu) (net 1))
 (segment (start 157.48 124.46) (end 161.29 124.46) (width 0.75) (layer F.Cu) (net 1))
 (segment (start 157.48 131.445) (end 157.48 124.46) (width 0.75) (layer F.Cu) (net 1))
 (via (at 157.48 131.445) (size 1.7) (drill 1) (layers F.Cu B.Cu) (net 1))
 (segment (start 152.4 133.985) (end 152.4 131.445) (width 0.75) (layer F.Cu) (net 1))
 (segment (start 156.1011 109.5036) (end 158.4664 109.5036) (width 0.75) (layer F.Cu) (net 1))
 (segment (start 158.4664 109.5036) (end 159.4528 110.49) (width 0.75) (layer F.Cu) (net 1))
 (segment (start 159.4528 110.49) (end 160.02 110.49) (width 0.75) (layer F.Cu) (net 1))
 (segment (start 156.1011 111.5036) (end 157.8586 111.5036) (width 0.75) (layer F.Cu) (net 17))
 (segment (start 157.8586 111.5036) (end 159.385 113.03) (width 0.75) (layer F.Cu) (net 17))
 (segment (start 159.385 113.03) (end 160.02 113.03) (width 0.75) (layer F.Cu) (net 17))
 (segment (start 160.02 115.57) (end 161.925 115.57) (width 0.75) (layer F.Cu) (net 3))
 (segment (start 161.925 119.38) (end 160.02 121.285) (width 0.75) (layer F.Cu) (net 3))
 (segment (start 161.925 115.57) (end 161.925 119.38) (width 0.75) (layer F.Cu) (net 3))
 (segment (start 156.1011 113.5036) (end 157.3186 113.5036) (width 0.75) (layer F.Cu) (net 3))
 (segment (start 157.3186 113.5036) (end 159.385 115.57) (width 0.75) (layer F.Cu) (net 3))
 (segment (start 159.385 115.57) (end 160.02 115.57) (width 0.75) (layer F.Cu) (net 3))
 (segment (start 147.32 133.985) (end 147.32 136.525) (width 0.75) (layer F.Cu) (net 13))
 (segment (start 161.29 100.33) (end 160.02 100.33) (width 0.75) (layer F.Cu) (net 13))
 (segment (start 165.735 104.775) (end 161.29 100.33) (width 0.75) (layer F.Cu) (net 13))
 (segment (start 165.735 125.73) (end 165.735 104.775) (width 0.75) (layer F.Cu) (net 13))
 (segment (start 163.195 128.27) (end 165.735 125.73) (width 0.75) (layer F.Cu) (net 13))
 (segment (start 163.195 132.08) (end 163.195 128.27) (width 0.75) (layer F.Cu) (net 13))
 (segment (start 162.56 132.715) (end 163.195 132.08) (width 0.75) (layer F.Cu) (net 13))
 (segment (start 161.29 132.715) (end 162.56 132.715) (width 0.75) (layer F.Cu) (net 13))
 (segment (start 157.48 136.525) (end 161.29 132.715) (width 0.75) (layer F.Cu) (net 13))
 (segment (start 147.32 136.525) (end 157.48 136.525) (width 0.75) (layer F.Cu) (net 13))
 (segment (start 156.1011 101.5036) (end 157.3836 101.5036) (width 0.75) (layer F.Cu) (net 13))
 (segment (start 158.5572 100.33) (end 160.02 100.33) (width 0.75) (layer F.Cu) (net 13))
 (segment (start 157.3836 101.5036) (end 158.5572 100.33) (width 0.75) (layer F.Cu) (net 13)))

